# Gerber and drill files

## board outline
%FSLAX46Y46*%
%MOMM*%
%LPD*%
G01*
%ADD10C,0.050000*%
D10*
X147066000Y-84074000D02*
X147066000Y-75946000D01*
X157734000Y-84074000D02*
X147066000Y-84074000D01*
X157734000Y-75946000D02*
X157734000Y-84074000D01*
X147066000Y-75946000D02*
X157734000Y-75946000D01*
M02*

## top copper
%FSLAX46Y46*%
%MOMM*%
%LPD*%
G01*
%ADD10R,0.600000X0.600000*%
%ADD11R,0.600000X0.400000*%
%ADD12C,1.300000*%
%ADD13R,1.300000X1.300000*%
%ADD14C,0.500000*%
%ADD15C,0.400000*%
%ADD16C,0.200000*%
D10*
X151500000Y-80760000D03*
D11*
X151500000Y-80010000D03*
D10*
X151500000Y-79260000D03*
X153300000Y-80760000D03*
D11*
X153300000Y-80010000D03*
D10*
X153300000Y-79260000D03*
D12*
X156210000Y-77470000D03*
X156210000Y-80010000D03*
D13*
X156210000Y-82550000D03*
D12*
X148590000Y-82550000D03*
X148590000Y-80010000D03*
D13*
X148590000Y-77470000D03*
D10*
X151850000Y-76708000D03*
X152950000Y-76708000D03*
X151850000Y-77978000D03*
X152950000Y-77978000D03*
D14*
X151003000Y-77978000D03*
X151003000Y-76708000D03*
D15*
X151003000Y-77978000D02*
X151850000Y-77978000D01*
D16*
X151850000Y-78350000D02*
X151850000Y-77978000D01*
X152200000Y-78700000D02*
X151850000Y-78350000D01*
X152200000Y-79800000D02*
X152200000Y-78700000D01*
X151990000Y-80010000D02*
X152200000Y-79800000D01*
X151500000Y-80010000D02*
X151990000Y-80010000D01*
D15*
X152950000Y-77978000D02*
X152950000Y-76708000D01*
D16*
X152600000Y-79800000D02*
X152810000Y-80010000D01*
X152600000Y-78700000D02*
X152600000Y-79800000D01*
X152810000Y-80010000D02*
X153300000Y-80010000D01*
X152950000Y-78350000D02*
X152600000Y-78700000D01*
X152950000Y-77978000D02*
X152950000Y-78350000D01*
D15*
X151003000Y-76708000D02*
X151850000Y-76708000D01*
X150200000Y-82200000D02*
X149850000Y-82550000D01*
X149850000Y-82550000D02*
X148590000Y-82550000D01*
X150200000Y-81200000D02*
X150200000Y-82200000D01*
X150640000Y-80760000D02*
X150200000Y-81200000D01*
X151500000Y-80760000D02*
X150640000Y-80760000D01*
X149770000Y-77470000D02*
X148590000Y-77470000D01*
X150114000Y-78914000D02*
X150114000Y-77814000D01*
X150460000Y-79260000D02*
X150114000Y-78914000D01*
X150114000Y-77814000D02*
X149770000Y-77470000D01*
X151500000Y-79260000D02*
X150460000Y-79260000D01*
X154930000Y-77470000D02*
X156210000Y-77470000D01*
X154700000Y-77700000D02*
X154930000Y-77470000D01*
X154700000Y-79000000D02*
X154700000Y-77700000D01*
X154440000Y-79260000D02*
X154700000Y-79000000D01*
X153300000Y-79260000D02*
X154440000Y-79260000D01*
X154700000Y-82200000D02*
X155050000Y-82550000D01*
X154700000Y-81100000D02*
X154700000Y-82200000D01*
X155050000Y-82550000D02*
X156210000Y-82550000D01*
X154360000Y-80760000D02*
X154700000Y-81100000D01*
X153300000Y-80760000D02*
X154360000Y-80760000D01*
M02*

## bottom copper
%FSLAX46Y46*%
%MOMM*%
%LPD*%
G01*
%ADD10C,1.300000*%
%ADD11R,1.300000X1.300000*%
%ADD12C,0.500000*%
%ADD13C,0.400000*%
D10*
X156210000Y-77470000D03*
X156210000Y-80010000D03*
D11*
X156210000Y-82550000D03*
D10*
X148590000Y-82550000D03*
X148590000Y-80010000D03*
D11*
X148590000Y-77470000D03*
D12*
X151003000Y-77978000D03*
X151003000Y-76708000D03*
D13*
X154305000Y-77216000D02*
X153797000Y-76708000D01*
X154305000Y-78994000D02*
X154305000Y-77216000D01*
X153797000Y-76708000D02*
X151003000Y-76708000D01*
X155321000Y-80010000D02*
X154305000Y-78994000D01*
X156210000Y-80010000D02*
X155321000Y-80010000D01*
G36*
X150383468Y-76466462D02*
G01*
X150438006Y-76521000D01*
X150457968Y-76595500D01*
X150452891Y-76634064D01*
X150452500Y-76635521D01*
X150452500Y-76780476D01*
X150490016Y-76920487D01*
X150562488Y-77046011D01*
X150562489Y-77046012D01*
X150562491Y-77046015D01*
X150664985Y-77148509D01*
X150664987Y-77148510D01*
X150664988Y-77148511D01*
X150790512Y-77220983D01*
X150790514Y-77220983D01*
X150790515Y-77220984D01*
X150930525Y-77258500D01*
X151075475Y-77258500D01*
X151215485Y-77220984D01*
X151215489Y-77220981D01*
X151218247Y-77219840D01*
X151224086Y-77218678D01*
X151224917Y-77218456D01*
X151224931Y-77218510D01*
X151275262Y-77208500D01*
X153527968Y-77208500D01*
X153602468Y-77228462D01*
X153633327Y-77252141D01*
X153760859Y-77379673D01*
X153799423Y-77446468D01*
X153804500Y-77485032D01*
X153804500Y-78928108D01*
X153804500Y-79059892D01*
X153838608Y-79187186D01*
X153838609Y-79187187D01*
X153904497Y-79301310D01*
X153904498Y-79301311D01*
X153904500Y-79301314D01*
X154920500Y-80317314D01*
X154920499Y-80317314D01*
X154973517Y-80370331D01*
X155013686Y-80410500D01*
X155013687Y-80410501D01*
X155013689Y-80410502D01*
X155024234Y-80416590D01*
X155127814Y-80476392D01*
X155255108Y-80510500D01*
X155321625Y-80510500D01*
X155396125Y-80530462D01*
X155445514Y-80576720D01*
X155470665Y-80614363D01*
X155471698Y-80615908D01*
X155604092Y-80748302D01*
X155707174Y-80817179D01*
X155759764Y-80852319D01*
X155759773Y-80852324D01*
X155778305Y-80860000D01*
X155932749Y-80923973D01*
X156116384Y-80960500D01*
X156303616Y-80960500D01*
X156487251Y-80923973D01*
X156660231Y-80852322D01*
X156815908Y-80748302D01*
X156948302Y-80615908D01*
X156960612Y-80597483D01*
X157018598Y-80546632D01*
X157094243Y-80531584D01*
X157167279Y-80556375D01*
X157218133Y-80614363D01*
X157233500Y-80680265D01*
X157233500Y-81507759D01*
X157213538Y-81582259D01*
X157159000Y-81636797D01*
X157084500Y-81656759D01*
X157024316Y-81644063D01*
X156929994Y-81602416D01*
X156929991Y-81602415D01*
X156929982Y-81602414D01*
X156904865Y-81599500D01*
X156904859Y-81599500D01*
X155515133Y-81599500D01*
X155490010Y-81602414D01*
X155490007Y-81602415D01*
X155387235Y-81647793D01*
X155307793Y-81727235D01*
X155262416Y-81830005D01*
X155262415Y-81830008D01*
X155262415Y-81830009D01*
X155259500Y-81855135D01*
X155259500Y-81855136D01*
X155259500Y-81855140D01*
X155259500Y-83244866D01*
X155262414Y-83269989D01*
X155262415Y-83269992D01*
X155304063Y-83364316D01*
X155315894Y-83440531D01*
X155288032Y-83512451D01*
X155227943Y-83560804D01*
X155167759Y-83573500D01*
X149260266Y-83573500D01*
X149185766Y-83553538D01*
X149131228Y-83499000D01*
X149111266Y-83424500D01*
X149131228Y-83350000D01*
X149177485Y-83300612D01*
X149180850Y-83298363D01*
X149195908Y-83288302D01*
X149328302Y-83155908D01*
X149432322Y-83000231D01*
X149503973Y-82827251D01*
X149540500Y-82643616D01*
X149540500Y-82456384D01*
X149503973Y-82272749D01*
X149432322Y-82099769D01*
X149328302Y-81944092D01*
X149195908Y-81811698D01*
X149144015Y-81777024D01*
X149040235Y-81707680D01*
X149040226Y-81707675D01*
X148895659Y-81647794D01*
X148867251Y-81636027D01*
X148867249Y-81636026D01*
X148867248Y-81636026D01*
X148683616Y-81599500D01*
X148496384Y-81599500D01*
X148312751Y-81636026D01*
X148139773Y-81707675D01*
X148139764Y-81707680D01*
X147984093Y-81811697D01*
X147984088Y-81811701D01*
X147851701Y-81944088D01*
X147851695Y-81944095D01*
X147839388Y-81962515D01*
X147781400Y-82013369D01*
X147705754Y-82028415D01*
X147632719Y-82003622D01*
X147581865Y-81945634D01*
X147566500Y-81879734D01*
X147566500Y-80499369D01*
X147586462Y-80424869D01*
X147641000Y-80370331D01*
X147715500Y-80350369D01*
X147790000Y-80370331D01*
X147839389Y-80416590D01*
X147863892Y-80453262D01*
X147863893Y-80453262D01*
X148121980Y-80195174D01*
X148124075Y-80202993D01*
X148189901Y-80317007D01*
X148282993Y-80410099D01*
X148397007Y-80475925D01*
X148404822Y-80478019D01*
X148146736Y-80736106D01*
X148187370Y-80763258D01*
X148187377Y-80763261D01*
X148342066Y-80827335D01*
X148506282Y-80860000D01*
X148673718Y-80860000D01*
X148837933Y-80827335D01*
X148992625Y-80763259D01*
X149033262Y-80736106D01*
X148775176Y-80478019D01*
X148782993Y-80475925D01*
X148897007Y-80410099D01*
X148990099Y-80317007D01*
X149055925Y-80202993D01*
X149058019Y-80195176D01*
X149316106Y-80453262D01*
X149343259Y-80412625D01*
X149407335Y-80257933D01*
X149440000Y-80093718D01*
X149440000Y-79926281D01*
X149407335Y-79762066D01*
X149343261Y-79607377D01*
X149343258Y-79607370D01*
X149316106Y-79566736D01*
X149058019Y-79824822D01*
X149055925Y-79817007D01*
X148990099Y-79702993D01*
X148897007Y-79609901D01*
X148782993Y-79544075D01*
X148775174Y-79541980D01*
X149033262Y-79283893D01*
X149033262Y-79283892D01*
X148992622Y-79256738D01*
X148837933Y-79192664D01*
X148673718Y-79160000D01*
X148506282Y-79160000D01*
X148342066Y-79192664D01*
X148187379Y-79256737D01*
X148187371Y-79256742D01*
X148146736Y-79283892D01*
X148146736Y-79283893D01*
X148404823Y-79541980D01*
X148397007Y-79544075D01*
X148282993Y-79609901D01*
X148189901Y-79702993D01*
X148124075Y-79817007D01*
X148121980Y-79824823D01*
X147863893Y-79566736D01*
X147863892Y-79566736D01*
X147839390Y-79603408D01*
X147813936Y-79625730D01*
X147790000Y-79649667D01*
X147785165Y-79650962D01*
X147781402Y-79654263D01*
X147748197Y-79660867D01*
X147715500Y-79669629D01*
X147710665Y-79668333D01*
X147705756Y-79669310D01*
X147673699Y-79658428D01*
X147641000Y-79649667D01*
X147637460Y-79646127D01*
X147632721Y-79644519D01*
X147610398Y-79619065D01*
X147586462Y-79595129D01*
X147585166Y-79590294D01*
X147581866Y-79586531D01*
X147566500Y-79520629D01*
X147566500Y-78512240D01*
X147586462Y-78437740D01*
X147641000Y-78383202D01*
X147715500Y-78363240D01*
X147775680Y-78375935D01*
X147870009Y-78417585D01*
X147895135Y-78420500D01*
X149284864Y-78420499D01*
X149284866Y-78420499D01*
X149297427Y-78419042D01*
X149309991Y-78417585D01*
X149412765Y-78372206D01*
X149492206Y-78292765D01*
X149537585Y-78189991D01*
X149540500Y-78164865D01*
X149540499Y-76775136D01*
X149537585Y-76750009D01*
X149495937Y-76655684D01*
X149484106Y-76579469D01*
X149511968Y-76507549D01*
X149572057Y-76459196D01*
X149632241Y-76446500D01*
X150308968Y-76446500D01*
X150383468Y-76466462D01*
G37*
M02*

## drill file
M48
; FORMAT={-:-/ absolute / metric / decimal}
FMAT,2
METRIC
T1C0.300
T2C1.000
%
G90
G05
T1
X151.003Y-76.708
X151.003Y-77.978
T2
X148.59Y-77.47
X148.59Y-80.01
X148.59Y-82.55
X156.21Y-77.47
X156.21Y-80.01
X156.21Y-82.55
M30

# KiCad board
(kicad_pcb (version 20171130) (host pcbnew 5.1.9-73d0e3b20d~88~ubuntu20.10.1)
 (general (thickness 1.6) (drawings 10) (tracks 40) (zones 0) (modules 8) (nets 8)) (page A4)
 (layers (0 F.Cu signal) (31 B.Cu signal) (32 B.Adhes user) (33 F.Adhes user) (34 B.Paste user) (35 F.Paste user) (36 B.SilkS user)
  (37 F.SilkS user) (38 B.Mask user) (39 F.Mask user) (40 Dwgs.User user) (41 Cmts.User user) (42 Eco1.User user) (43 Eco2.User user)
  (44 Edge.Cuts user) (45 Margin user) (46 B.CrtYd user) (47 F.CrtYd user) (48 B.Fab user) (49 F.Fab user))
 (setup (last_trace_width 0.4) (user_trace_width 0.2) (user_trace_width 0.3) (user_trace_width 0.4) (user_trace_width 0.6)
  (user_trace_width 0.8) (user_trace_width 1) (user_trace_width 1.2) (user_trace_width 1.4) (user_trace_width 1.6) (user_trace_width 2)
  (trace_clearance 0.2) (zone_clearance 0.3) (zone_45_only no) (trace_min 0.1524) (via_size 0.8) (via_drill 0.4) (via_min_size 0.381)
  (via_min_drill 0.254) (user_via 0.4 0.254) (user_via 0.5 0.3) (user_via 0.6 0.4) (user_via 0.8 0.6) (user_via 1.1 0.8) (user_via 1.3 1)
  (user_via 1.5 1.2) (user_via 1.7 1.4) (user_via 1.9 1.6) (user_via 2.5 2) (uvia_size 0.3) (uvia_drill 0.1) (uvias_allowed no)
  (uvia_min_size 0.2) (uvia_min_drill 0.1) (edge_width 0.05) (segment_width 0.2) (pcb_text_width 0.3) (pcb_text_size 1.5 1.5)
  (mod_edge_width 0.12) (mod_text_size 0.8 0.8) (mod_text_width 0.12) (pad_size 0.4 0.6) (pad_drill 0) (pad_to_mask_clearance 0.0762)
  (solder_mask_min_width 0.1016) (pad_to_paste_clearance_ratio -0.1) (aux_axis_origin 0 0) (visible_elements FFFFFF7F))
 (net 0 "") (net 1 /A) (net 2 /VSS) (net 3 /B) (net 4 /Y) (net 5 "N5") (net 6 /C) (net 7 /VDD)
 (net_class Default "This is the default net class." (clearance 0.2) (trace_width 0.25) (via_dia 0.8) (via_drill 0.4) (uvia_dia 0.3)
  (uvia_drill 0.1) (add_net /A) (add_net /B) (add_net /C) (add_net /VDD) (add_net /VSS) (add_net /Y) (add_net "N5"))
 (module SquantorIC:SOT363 (layer F.Cu) (at 152.4 80.01 270)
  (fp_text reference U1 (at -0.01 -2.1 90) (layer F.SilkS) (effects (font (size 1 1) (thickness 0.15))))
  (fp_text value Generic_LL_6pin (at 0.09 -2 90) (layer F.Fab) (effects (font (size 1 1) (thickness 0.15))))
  (pad 3 smd rect (at 0.75 0.9 270) (size 0.6 0.6) (layers F.Cu F.Paste F.Mask) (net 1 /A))
  (pad 2 smd rect (at 0 0.9 270) (size 0.4 0.6) (layers F.Cu F.Paste F.Mask) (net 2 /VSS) (zone_connect 2))
  (pad 1 smd rect (at -0.75 0.9 270) (size 0.6 0.6) (layers F.Cu F.Paste F.Mask) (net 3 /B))
  (pad 4 smd rect (at 0.75 -0.9 270) (size 0.6 0.6) (layers F.Cu F.Paste F.Mask) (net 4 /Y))
  (pad 5 smd rect (at 0 -0.9 270) (size 0.4 0.6) (layers F.Cu F.Paste F.Mask) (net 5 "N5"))
  (pad 6 smd rect (at -0.75 -0.9 270) (size 0.6 0.6) (layers F.Cu F.Paste F.Mask) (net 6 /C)))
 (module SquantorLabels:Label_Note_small (layer F.Cu) (at 149.352 82.55)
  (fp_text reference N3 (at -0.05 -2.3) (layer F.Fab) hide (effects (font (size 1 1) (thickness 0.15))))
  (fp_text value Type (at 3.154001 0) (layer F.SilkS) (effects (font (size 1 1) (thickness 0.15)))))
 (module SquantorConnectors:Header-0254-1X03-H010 (layer B.Cu) (at 156.21 80.01 90)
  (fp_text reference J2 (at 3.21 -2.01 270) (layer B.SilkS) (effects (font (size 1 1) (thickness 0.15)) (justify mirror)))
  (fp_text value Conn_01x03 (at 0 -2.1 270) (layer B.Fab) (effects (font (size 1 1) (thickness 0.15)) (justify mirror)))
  (pad 3 thru_hole circle (at 2.54 0 270) (size 1.3 1.3) (drill 1) (layers *.Cu *.Mask) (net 6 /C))
  (pad 2 thru_hole circle (at 0 0 270) (size 1.3 1.3) (drill 1) (layers *.Cu *.Mask) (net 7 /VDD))
  (pad 1 thru_hole rect (at -2.54 0 270) (size 1.3 1.3) (drill 1) (layers *.Cu *.Mask) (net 4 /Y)))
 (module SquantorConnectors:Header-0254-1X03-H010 (layer B.Cu) (at 148.59 80.01 270)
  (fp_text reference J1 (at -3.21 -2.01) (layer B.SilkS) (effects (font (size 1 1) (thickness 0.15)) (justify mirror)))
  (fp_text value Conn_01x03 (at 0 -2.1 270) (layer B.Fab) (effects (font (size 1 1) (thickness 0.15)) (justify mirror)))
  (pad 3 thru_hole circle (at 2.54 0 90) (size 1.3 1.3) (drill 1) (layers *.Cu *.Mask) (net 1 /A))
  (pad 2 thru_hole circle (at 0 0 90) (size 1.3 1.3) (drill 1) (layers *.Cu *.Mask) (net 2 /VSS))
  (pad 1 thru_hole rect (at -2.54 0 90) (size 1.3 1.3) (drill 1) (layers *.Cu *.Mask) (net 3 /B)))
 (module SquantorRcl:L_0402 (layer F.Cu) (at 152.4 76.708 180)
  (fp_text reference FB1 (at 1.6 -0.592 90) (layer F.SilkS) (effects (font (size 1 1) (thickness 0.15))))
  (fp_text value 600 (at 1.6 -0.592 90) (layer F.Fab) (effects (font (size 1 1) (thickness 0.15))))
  (pad 2 smd rect (at 0.55 0 180) (size 0.6 0.6) (layers F.Cu F.Paste F.Mask) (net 7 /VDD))
  (pad 1 smd rect (at -0.55 0 180) (size 0.6 0.6) (layers F.Cu F.Paste F.Mask) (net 5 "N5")))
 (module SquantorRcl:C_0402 (layer F.Cu) (at 152.4 77.978 180) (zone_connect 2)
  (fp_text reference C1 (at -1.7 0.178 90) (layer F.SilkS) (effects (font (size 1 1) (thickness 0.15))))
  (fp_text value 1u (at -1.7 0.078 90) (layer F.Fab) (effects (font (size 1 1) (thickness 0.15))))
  (pad 2 smd rect (at 0.55 0 180) (size 0.6 0.6) (layers F.Cu F.Paste F.Mask) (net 2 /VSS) (zone_connect 2))
  (pad 1 smd rect (at -0.55 0 180) (size 0.6 0.6) (layers F.Cu F.Paste F.Mask) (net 5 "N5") (zone_connect 2)))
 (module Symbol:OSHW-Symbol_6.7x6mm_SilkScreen (layer B.Cu) (at 152.4 79.7 180)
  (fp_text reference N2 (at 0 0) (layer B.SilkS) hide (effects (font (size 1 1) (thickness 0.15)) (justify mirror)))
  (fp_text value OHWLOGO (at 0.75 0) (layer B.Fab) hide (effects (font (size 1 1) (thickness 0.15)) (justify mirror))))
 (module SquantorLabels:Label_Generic (layer B.Cu) (at 153.162 83.312 180)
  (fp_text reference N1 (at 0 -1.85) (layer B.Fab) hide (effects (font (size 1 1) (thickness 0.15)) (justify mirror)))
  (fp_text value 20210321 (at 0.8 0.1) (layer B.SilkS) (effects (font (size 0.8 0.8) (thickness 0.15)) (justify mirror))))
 (gr_line (start 147.066 84.074) (end 147.066 75.946) (layer Edge.Cuts) (width 0.05))
 (gr_line (start 157.734 84.074) (end 147.066 84.074) (layer Edge.Cuts) (width 0.05))
 (gr_line (start 157.734 75.946) (end 157.734 84.074) (layer Edge.Cuts) (width 0.05))
 (gr_line (start 147.066 75.946) (end 157.734 75.946) (layer Edge.Cuts) (width 0.05))
 (via (at 151.003 77.978) (size 0.5) (drill 0.3) (layers F.Cu B.Cu) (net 2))
 (segment (start 151.003 77.978) (end 151.85 77.978) (width 0.4) (layer F.Cu) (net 2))
 (segment (start 151.85 78.35) (end 151.85 77.978) (width 0.2) (layer F.Cu) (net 2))
 (segment (start 152.2 78.7) (end 151.85 78.35) (width 0.2) (layer F.Cu) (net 2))
 (segment (start 152.2 79.8) (end 152.2 78.7) (width 0.2) (layer F.Cu) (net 2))
 (segment (start 151.99 80.01) (end 152.2 79.8) (width 0.2) (layer F.Cu) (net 2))
 (segment (start 151.5 80.01) (end 151.99 80.01) (width 0.2) (layer F.Cu) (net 2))
 (segment (start 152.95 77.978) (end 152.95 76.708) (width 0.4) (layer F.Cu) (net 5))
 (segment (start 152.6 79.8) (end 152.81 80.01) (width 0.2) (layer F.Cu) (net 5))
 (segment (start 152.6 78.7) (end 152.6 79.8) (width 0.2) (layer F.Cu) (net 5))
 (segment (start 152.81 80.01) (end 153.3 80.01) (width 0.2) (layer F.Cu) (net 5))
 (segment (start 152.95 78.35) (end 152.6 78.7) (width 0.2) (layer F.Cu) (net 5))
 (segment (start 152.95 77.978) (end 152.95 78.35) (width 0.2) (layer F.Cu) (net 5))
 (via (at 151.003 76.708) (size 0.5) (drill 0.3) (layers F.Cu B.Cu) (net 7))
 (segment (start 151.003 76.708) (end 151.85 76.708) (width 0.4) (layer F.Cu) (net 7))
 (segment (start 154.305 77.216) (end 153.797 76.708) (width 0.4) (layer B.Cu) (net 7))
 (segment (start 154.305 78.994) (end 154.305 77.216) (width 0.4) (layer B.Cu) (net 7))
 (segment (start 153.797 76.708) (end 151.003 76.708) (width 0.4) (layer B.Cu) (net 7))
 (segment (start 155.321 80.01) (end 154.305 78.994) (width 0.4) (layer B.Cu) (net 7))
 (segment (start 156.21 80.01) (end 155.321 80.01) (width 0.4) (layer B.Cu) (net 7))
 (segment (start 150.2 82.2) (end 149.85 82.55) (width 0.4) (layer F.Cu) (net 1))
 (segment (start 149.85 82.55) (end 148.59 82.55) (width 0.4) (layer F.Cu) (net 1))
 (segment (start 150.2 81.2) (end 150.2 82.2) (width 0.4) (layer F.Cu) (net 1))
 (segment (start 150.64 80.76) (end 150.2 81.2) (width 0.4) (layer F.Cu) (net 1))
 (segment (start 151.5 80.76) (end 150.64 80.76) (width 0.4) (layer F.Cu) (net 1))
 (segment (start 149.77 77.47) (end 148.59 77.47) (width 0.4) (layer F.Cu) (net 3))
 (segment (start 150.114 78.914) (end 150.114 77.814) (width 0.4) (layer F.Cu) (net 3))
 (segment (start 150.46 79.26) (end 150.114 78.914) (width 0.4) (layer F.Cu) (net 3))
 (segment (start 150.114 77.814) (end 149.77 77.47) (width 0.4) (layer F.Cu) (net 3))
 (segment (start 151.5 79.26) (end 150.46 79.26) (width 0.4) (layer F.Cu) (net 3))
 (segment (start 154.93 77.47) (end 156.21 77.47) (width 0.4) (layer F.Cu) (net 6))
 (segment (start 154.7 77.7) (end 154.93 77.47) (width 0.4) (layer F.Cu) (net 6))
 (segment (start 154.7 79) (end 154.7 77.7) (width 0.4) (layer F.Cu) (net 6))
 (segment (start 154.44 79.26) (end 154.7 79) (width 0.4) (layer F.Cu) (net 6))
 (segment (start 153.3 79.26) (end 154.44 79.26) (width 0.4) (layer F.Cu) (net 6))
 (segment (start 154.7 82.2) (end 155.05 82.55) (width 0.4) (layer F.Cu) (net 4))
 (segment (start 154.7 81.1) (end 154.7 82.2) (width 0.4) (layer F.Cu) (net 4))
 (segment (start 155.05 82.55) (end 156.21 82.55) (width 0.4) (layer F.Cu) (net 4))
 (segment (start 154.36 80.76) (end 154.7 81.1) (width 0.4) (layer F.Cu) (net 4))
 (segment (start 153.3 80.76) (end 154.36 80.76) (width 0.4) (layer F.Cu) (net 4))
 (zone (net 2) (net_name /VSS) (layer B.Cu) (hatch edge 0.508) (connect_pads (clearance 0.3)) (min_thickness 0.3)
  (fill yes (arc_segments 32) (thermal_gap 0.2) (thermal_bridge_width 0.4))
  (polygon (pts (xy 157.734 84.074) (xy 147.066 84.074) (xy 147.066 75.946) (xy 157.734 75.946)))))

